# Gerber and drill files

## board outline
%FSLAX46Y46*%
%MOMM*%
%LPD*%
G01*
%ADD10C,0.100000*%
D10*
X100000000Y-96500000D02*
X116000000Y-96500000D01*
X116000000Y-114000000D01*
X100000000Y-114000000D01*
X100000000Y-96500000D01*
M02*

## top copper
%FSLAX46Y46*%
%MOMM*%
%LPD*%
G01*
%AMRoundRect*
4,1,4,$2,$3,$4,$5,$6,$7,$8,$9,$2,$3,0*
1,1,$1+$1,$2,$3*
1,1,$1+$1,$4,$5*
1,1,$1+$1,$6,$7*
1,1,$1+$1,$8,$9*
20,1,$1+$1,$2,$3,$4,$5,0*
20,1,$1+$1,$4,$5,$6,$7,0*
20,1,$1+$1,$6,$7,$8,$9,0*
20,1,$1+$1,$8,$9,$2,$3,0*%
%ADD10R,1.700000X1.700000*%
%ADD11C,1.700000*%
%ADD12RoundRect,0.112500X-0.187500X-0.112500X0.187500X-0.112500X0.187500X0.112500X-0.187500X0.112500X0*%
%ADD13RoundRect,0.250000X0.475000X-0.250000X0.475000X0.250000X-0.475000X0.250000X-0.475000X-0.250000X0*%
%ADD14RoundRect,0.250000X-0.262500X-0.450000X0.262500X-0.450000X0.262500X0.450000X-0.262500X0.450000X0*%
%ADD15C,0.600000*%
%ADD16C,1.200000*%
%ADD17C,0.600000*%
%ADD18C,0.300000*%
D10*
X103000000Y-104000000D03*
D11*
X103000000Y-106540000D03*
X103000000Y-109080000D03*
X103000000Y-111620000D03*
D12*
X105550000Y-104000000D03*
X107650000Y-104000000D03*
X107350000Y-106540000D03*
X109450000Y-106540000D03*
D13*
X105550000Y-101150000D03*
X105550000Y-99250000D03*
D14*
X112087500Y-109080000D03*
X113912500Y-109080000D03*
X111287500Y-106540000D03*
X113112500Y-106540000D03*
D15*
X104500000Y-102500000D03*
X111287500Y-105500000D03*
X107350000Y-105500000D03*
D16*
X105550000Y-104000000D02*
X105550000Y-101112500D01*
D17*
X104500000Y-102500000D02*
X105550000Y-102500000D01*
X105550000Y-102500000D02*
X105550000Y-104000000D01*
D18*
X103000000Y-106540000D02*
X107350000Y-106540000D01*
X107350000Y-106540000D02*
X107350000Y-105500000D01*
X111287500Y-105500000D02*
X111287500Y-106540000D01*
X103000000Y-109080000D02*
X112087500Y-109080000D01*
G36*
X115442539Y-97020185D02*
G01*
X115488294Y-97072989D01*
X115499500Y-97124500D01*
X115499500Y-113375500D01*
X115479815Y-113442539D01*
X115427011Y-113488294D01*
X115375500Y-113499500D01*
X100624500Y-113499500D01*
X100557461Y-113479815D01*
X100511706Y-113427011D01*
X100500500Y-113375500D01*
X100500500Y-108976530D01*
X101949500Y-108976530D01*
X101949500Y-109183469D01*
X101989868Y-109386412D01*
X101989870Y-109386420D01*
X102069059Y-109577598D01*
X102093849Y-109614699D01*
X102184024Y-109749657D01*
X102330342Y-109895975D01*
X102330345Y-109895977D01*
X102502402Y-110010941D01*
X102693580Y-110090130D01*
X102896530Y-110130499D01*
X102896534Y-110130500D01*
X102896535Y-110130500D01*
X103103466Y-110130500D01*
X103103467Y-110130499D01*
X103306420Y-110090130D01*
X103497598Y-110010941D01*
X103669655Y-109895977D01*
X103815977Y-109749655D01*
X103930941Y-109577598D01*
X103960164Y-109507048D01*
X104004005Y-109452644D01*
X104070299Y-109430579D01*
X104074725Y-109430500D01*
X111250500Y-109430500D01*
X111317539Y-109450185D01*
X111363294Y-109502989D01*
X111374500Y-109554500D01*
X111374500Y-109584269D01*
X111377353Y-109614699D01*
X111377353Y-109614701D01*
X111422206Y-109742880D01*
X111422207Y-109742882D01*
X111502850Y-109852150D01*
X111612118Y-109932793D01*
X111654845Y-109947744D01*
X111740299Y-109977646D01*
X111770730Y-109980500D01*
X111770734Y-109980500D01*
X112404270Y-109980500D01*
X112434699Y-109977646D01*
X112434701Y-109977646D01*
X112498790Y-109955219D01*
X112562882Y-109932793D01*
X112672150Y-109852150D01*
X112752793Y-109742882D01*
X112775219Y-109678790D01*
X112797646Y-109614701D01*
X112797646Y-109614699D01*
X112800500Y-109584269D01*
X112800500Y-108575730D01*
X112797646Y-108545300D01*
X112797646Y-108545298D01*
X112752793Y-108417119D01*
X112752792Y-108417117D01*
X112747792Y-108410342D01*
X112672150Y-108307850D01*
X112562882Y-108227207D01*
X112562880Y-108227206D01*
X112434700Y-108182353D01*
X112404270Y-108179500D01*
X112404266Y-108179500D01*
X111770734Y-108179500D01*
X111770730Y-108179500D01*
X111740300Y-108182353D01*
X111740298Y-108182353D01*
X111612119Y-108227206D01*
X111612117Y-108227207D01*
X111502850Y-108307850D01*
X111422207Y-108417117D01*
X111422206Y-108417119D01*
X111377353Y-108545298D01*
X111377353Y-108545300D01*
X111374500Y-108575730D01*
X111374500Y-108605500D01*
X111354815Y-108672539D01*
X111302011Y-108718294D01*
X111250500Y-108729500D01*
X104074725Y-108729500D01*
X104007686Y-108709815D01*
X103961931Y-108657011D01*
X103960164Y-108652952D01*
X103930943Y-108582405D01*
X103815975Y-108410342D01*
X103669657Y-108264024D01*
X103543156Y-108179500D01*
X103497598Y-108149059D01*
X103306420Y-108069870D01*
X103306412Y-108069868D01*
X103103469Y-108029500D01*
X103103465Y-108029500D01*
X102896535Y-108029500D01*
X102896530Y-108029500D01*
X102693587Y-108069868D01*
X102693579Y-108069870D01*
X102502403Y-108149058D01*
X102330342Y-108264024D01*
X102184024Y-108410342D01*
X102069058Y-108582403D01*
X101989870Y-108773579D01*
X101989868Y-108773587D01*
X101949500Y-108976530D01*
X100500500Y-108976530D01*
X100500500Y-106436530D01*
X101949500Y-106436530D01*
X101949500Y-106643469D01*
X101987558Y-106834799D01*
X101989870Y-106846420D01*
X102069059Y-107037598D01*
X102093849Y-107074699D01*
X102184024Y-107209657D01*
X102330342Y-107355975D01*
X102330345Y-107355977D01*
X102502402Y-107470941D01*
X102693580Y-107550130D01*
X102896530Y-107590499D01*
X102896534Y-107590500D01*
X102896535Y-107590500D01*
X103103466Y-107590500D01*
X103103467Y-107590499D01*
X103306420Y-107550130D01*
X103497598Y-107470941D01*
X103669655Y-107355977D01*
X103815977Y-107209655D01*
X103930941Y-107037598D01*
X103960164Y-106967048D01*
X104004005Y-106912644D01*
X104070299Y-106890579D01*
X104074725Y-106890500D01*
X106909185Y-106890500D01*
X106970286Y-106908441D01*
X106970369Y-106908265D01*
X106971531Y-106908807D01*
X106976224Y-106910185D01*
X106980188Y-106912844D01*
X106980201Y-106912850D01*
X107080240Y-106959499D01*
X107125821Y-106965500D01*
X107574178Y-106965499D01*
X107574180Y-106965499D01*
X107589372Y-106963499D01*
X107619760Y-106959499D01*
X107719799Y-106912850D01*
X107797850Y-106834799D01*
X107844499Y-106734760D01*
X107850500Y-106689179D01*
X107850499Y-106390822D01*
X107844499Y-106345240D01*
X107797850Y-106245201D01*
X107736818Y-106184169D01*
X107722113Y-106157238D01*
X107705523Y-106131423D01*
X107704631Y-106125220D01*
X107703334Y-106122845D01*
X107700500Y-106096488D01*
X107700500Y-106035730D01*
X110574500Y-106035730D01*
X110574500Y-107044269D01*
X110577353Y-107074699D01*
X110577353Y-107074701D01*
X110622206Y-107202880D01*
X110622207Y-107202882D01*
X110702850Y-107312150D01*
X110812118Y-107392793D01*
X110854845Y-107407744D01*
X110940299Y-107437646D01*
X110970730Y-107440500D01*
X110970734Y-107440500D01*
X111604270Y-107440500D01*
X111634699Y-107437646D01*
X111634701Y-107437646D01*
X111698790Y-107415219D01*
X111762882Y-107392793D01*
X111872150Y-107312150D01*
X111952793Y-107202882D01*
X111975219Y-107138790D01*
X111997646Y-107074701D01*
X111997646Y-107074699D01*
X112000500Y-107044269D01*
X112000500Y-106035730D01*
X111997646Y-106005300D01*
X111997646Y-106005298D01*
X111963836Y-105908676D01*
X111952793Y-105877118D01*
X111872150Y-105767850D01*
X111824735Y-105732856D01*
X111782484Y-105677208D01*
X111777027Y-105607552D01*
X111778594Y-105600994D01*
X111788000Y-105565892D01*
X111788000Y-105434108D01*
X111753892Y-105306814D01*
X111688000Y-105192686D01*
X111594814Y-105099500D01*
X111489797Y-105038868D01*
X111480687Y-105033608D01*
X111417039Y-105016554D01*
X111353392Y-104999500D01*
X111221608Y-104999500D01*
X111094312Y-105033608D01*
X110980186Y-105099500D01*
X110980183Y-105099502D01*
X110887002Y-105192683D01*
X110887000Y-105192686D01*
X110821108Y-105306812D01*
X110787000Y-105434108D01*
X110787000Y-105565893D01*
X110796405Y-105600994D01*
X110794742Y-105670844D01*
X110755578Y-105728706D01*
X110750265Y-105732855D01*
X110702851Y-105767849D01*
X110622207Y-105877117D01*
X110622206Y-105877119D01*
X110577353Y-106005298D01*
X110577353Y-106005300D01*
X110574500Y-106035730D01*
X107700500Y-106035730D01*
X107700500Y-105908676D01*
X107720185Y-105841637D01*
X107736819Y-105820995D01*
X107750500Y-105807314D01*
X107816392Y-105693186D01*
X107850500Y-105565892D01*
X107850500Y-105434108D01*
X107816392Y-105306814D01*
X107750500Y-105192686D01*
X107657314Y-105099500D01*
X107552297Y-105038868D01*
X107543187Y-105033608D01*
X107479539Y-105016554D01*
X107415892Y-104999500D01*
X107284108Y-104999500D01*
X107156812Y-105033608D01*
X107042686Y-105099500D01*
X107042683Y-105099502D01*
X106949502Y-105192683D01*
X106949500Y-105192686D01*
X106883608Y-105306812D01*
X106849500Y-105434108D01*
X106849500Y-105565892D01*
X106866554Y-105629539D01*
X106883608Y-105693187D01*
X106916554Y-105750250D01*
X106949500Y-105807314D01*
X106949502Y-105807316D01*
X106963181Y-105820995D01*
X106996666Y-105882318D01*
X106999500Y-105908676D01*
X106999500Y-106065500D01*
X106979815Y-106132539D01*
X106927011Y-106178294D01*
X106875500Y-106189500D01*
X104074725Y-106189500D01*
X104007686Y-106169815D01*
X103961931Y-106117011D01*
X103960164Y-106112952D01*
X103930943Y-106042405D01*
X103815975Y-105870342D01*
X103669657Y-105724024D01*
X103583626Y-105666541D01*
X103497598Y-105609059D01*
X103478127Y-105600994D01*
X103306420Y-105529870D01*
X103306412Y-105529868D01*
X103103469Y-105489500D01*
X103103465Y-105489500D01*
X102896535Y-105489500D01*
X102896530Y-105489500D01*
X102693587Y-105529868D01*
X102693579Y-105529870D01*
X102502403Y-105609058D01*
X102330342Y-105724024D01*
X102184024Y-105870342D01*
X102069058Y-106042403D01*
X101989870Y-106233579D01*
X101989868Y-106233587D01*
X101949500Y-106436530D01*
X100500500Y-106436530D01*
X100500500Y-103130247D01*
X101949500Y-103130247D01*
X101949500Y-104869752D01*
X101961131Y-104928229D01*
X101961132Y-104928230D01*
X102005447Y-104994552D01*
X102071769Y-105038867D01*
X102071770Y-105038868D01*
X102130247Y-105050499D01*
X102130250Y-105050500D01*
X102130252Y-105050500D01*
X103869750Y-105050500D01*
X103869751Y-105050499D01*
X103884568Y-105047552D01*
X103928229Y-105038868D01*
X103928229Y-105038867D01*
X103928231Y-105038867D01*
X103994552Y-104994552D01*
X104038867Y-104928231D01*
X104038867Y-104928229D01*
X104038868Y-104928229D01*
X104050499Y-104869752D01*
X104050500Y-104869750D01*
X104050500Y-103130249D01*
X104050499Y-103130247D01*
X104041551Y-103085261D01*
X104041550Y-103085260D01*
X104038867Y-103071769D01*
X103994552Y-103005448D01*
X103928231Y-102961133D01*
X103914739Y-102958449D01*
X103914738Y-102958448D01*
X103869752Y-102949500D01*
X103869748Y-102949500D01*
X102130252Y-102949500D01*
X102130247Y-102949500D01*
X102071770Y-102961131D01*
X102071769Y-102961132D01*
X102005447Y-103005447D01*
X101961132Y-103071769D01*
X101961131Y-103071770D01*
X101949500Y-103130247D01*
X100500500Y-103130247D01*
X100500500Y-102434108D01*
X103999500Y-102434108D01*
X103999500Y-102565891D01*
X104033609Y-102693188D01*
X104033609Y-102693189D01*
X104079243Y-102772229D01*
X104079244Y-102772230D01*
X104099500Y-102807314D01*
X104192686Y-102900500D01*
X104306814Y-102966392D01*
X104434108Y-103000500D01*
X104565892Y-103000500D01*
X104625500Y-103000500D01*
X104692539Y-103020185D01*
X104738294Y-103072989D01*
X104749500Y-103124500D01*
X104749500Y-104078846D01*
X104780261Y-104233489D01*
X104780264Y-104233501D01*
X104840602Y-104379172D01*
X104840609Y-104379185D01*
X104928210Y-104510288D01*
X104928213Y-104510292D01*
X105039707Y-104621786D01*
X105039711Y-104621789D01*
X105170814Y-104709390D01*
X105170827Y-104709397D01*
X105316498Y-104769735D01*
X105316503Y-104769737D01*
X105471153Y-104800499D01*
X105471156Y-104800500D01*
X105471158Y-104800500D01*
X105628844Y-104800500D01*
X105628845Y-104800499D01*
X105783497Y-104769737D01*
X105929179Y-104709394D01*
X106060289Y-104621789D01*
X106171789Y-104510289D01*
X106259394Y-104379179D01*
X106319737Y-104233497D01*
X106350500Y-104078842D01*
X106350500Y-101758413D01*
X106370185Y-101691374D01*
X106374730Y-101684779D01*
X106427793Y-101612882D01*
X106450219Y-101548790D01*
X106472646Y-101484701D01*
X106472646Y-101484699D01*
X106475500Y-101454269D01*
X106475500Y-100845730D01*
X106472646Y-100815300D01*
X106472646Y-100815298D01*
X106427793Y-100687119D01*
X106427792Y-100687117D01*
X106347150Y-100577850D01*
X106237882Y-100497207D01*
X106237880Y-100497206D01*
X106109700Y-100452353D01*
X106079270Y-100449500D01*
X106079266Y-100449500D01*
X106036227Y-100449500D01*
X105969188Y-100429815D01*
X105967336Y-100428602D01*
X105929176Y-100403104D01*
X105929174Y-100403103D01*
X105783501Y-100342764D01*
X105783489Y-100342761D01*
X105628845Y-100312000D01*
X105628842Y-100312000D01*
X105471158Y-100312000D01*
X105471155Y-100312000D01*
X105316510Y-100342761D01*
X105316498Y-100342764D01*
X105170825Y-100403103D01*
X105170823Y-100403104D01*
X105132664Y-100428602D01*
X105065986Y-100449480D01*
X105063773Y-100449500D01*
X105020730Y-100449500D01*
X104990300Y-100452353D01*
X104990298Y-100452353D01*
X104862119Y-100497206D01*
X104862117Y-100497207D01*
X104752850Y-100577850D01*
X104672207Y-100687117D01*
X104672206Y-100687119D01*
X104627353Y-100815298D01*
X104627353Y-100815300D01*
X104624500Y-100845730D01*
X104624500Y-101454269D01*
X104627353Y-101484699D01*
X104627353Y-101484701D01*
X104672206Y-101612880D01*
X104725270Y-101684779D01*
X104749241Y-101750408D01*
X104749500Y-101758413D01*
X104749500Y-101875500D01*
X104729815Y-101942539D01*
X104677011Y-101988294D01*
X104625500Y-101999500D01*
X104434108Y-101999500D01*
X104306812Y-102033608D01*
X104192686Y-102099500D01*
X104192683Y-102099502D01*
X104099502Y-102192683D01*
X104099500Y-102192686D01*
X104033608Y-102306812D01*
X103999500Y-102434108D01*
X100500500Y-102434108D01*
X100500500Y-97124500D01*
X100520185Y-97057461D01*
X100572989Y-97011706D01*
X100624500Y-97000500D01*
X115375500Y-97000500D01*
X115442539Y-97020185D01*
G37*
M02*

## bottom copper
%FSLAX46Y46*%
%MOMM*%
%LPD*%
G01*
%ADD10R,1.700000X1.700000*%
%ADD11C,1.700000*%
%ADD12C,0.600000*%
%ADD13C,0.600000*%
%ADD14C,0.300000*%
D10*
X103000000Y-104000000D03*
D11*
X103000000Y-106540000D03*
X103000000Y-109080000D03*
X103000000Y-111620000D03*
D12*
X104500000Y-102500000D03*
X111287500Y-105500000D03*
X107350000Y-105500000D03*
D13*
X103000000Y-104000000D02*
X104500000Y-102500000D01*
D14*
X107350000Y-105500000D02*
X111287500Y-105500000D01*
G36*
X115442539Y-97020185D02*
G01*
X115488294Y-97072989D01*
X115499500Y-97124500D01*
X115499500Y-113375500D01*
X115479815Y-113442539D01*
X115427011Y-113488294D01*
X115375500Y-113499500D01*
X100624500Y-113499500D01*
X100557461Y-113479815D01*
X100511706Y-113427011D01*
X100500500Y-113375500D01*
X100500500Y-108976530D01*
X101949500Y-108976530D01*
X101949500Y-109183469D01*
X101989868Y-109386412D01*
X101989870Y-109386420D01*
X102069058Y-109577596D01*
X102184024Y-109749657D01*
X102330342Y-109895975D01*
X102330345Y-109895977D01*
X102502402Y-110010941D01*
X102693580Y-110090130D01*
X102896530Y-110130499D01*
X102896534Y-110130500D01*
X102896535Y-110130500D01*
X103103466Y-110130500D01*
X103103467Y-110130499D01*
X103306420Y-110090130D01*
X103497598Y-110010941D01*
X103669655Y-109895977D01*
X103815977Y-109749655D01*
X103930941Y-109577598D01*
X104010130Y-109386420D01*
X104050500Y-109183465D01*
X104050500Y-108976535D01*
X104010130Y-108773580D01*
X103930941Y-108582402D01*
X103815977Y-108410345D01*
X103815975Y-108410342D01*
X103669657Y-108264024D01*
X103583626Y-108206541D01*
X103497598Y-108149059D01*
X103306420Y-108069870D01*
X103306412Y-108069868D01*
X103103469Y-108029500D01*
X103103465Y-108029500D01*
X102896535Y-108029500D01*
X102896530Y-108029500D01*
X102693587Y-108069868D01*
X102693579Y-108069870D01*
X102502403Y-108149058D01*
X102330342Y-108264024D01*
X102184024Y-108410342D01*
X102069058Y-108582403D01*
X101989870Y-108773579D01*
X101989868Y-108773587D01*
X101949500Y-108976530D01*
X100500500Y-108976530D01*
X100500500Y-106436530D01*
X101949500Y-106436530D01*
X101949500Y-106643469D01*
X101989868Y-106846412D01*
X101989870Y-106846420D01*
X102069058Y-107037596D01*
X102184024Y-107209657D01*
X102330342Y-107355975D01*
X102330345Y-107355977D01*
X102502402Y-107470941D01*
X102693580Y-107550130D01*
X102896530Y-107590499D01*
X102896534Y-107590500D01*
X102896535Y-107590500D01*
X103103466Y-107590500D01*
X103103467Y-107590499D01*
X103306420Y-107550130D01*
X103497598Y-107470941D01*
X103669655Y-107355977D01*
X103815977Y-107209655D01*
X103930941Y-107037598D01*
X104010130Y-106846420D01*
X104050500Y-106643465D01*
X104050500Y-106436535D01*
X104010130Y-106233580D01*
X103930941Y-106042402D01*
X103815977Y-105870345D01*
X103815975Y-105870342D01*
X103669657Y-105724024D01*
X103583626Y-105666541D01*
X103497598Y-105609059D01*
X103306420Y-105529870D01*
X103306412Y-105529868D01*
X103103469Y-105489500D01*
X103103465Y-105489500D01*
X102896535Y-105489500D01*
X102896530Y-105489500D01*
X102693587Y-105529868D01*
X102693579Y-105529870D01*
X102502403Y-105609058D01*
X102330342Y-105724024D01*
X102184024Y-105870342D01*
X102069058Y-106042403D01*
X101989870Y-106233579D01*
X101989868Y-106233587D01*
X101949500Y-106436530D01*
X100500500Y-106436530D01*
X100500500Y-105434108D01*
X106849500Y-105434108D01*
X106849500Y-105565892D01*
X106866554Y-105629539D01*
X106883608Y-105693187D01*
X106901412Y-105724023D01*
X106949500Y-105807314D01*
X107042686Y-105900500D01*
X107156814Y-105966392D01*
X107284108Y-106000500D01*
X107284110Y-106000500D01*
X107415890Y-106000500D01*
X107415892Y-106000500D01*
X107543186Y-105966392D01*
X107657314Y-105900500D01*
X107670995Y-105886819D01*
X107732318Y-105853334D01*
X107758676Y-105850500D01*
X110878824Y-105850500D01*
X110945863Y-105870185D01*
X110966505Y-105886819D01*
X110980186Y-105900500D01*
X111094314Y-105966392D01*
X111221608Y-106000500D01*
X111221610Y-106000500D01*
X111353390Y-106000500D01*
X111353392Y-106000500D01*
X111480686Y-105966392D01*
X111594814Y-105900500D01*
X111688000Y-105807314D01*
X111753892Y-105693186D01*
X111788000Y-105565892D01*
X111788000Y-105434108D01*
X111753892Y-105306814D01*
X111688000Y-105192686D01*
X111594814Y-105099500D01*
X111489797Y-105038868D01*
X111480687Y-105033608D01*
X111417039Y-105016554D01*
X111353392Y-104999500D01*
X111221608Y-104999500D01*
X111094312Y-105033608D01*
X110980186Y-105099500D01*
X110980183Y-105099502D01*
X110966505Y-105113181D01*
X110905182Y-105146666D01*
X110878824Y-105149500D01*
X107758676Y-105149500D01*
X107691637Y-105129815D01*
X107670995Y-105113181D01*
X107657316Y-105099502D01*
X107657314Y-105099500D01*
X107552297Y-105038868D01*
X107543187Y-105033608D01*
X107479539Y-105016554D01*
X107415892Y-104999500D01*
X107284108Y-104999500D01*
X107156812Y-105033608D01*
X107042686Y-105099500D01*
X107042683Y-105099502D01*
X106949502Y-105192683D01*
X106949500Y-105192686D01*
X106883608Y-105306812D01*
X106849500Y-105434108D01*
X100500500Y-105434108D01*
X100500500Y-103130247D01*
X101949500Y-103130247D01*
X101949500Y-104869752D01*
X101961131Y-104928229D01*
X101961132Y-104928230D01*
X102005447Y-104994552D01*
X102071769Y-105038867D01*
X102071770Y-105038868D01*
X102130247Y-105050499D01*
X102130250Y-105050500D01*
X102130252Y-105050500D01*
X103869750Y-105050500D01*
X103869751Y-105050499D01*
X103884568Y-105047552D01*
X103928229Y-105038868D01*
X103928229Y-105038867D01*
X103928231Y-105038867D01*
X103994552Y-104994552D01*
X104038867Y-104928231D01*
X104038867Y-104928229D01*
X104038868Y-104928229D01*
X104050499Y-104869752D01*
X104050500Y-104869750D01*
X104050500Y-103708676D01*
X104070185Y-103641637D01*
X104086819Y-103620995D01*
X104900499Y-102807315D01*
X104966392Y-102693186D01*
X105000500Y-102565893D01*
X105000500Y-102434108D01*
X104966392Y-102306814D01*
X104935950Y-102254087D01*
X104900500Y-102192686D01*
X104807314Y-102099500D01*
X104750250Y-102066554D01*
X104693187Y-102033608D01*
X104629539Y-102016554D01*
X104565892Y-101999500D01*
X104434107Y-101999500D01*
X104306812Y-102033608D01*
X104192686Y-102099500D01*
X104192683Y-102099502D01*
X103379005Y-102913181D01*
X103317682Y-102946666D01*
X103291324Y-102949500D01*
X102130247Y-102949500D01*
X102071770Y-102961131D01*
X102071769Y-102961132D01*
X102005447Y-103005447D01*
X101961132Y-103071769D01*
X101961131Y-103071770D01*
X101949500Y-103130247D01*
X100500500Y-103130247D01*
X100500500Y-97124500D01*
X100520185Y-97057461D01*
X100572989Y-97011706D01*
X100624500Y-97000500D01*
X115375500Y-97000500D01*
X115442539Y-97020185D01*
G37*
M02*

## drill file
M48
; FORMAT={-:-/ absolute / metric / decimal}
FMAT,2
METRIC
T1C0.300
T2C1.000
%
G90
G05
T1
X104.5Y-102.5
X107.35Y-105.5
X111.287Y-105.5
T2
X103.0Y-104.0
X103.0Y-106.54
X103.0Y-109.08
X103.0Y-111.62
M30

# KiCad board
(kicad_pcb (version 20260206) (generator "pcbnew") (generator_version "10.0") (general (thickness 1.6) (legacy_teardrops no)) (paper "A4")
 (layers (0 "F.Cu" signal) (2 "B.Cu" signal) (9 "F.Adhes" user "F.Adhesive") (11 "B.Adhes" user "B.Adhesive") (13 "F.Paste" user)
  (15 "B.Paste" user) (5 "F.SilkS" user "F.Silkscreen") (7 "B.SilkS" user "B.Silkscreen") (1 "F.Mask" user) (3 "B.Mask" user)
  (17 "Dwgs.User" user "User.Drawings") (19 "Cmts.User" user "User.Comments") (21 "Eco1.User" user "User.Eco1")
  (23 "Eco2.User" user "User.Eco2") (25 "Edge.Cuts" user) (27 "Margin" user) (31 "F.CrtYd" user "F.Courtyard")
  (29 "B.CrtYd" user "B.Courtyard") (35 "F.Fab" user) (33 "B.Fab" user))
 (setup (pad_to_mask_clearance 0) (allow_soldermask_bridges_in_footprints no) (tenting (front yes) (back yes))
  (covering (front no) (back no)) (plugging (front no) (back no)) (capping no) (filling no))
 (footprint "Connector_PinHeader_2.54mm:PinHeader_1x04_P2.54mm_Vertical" (layer "F.Cu") (at 103 104)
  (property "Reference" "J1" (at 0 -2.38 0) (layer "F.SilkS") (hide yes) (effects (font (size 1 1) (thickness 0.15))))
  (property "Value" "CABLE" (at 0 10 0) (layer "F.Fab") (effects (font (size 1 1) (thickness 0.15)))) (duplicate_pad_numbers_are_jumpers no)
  (pad "1" thru_hole rect (at 0 0) (size 1.7 1.7) (drill 1) (layers "*.Cu" "*.Mask") (remove_unused_layers no) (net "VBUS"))
  (pad "2" thru_hole circle (at 0 2.54) (size 1.7 1.7) (drill 1) (layers "*.Cu" "*.Mask") (remove_unused_layers no) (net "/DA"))
  (pad "3" thru_hole circle (at 0 5.08) (size 1.7 1.7) (drill 1) (layers "*.Cu" "*.Mask") (remove_unused_layers no) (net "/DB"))
  (pad "4" thru_hole circle (at 0 7.62) (size 1.7 1.7) (drill 1) (layers "*.Cu" "*.Mask") (remove_unused_layers no) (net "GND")))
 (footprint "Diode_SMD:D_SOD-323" (layer "F.Cu") (at 106.6 104)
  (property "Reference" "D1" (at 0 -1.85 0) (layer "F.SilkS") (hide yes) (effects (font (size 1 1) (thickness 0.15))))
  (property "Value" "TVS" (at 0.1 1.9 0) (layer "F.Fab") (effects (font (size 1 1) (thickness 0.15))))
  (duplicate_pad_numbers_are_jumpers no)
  (pad "1" smd roundrect (at -1.05 0) (size 0.6 0.45) (layers "F.Cu" "F.Mask" "F.Paste") (roundrect_rratio 0.25) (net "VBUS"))
  (pad "2" smd roundrect (at 1.05 0) (size 0.6 0.45) (layers "F.Cu" "F.Mask" "F.Paste") (roundrect_rratio 0.25) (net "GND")))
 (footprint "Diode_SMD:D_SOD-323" (layer "F.Cu") (at 108.4 106.54)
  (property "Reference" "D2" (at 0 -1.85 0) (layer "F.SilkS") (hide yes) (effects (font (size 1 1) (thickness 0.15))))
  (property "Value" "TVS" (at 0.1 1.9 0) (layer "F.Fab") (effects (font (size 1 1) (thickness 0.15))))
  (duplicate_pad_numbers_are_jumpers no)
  (pad "1" smd roundrect (at -1.05 0) (size 0.6 0.45) (layers "F.Cu" "F.Mask" "F.Paste") (roundrect_rratio 0.25) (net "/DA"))
  (pad "2" smd roundrect (at 1.05 0) (size 0.6 0.45) (layers "F.Cu" "F.Mask" "F.Paste") (roundrect_rratio 0.25) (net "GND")))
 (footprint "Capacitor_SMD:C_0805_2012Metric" (layer "F.Cu") (at 105.55 100.2 90)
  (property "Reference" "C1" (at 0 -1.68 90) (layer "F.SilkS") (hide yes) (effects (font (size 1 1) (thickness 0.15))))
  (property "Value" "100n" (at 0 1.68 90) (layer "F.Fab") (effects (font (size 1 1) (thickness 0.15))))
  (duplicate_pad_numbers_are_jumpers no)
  (pad "1" smd roundrect (at -0.95 0 90) (size 1 1.45) (layers "F.Cu" "F.Mask" "F.Paste") (roundrect_rratio 0.25) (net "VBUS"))
  (pad "2" smd roundrect (at 0.95 0 90) (size 1 1.45) (layers "F.Cu" "F.Mask" "F.Paste") (roundrect_rratio 0.25) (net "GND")))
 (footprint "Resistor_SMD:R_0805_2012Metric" (layer "F.Cu") (at 113 109.08)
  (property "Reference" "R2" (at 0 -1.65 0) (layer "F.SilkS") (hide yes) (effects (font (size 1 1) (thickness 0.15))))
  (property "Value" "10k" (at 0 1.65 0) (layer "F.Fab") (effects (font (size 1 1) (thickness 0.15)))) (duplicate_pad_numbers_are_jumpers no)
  (pad "1" smd roundrect (at -0.9125 0) (size 1.025 1.4) (layers "F.Cu" "F.Mask" "F.Paste") (roundrect_rratio 0.243902) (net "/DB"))
  (pad "2" smd roundrect (at 0.9125 0) (size 1.025 1.4) (layers "F.Cu" "F.Mask" "F.Paste") (roundrect_rratio 0.243902) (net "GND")))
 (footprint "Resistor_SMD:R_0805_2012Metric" (layer "F.Cu") (at 112.2 106.54)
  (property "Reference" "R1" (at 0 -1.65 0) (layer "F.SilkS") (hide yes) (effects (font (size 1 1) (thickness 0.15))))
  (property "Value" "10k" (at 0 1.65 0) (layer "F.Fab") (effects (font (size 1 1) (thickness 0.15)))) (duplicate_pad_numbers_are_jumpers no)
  (pad "1" smd roundrect (at -0.9125 0) (size 1.025 1.4) (layers "F.Cu" "F.Mask" "F.Paste") (roundrect_rratio 0.243902) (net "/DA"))
  (pad "2" smd roundrect (at 0.9125 0) (size 1.025 1.4) (layers "F.Cu" "F.Mask" "F.Paste") (roundrect_rratio 0.243902) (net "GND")))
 (gr_rect (start 100 96.5) (end 116 114) (stroke (width 0.1) (type default)) (fill no) (layer "Edge.Cuts"))
 (segment (start 105.55 104) (end 105.55 101.1125) (width 1.2) (layer "F.Cu") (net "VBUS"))
 (segment (start 104.5 102.5) (end 105.55 102.5) (width 0.6) (layer "F.Cu") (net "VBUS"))
 (segment (start 105.55 102.5) (end 105.55 104) (width 0.6) (layer "F.Cu") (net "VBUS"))
 (via (at 104.5 102.5) (size 0.6) (drill 0.3) (layers "F.Cu" "B.Cu") (capping no) (covering (front no) (back no))
  (plugging (front no) (back no)) (filling no) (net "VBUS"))
 (segment (start 103 104) (end 104.5 102.5) (width 0.6) (layer "B.Cu") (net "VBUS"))
 (segment (start 103 106.54) (end 107.35 106.54) (width 0.3) (layer "F.Cu") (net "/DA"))
 (segment (start 107.35 106.54) (end 107.35 105.5) (width 0.3) (layer "F.Cu") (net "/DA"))
 (segment (start 111.2875 105.5) (end 111.2875 106.54) (width 0.3) (layer "F.Cu") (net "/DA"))
 (via (at 111.2875 105.5) (size 0.6) (drill 0.3) (layers "F.Cu" "B.Cu") (capping no) (covering (front no) (back no))
  (plugging (front no) (back no)) (filling no) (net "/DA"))
 (via (at 107.35 105.5) (size 0.6) (drill 0.3) (layers "F.Cu" "B.Cu") (capping no) (covering (front no) (back no))
  (plugging (front no) (back no)) (filling no) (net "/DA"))
 (segment (start 107.35 105.5) (end 111.2875 105.5) (width 0.3) (layer "B.Cu") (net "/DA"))
 (segment (start 103 109.08) (end 112.0875 109.08) (width 0.3) (layer "F.Cu") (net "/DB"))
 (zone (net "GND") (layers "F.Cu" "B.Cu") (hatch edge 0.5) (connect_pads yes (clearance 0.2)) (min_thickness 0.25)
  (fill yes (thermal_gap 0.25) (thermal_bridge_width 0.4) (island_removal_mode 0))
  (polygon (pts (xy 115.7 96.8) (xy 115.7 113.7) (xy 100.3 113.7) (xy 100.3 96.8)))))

